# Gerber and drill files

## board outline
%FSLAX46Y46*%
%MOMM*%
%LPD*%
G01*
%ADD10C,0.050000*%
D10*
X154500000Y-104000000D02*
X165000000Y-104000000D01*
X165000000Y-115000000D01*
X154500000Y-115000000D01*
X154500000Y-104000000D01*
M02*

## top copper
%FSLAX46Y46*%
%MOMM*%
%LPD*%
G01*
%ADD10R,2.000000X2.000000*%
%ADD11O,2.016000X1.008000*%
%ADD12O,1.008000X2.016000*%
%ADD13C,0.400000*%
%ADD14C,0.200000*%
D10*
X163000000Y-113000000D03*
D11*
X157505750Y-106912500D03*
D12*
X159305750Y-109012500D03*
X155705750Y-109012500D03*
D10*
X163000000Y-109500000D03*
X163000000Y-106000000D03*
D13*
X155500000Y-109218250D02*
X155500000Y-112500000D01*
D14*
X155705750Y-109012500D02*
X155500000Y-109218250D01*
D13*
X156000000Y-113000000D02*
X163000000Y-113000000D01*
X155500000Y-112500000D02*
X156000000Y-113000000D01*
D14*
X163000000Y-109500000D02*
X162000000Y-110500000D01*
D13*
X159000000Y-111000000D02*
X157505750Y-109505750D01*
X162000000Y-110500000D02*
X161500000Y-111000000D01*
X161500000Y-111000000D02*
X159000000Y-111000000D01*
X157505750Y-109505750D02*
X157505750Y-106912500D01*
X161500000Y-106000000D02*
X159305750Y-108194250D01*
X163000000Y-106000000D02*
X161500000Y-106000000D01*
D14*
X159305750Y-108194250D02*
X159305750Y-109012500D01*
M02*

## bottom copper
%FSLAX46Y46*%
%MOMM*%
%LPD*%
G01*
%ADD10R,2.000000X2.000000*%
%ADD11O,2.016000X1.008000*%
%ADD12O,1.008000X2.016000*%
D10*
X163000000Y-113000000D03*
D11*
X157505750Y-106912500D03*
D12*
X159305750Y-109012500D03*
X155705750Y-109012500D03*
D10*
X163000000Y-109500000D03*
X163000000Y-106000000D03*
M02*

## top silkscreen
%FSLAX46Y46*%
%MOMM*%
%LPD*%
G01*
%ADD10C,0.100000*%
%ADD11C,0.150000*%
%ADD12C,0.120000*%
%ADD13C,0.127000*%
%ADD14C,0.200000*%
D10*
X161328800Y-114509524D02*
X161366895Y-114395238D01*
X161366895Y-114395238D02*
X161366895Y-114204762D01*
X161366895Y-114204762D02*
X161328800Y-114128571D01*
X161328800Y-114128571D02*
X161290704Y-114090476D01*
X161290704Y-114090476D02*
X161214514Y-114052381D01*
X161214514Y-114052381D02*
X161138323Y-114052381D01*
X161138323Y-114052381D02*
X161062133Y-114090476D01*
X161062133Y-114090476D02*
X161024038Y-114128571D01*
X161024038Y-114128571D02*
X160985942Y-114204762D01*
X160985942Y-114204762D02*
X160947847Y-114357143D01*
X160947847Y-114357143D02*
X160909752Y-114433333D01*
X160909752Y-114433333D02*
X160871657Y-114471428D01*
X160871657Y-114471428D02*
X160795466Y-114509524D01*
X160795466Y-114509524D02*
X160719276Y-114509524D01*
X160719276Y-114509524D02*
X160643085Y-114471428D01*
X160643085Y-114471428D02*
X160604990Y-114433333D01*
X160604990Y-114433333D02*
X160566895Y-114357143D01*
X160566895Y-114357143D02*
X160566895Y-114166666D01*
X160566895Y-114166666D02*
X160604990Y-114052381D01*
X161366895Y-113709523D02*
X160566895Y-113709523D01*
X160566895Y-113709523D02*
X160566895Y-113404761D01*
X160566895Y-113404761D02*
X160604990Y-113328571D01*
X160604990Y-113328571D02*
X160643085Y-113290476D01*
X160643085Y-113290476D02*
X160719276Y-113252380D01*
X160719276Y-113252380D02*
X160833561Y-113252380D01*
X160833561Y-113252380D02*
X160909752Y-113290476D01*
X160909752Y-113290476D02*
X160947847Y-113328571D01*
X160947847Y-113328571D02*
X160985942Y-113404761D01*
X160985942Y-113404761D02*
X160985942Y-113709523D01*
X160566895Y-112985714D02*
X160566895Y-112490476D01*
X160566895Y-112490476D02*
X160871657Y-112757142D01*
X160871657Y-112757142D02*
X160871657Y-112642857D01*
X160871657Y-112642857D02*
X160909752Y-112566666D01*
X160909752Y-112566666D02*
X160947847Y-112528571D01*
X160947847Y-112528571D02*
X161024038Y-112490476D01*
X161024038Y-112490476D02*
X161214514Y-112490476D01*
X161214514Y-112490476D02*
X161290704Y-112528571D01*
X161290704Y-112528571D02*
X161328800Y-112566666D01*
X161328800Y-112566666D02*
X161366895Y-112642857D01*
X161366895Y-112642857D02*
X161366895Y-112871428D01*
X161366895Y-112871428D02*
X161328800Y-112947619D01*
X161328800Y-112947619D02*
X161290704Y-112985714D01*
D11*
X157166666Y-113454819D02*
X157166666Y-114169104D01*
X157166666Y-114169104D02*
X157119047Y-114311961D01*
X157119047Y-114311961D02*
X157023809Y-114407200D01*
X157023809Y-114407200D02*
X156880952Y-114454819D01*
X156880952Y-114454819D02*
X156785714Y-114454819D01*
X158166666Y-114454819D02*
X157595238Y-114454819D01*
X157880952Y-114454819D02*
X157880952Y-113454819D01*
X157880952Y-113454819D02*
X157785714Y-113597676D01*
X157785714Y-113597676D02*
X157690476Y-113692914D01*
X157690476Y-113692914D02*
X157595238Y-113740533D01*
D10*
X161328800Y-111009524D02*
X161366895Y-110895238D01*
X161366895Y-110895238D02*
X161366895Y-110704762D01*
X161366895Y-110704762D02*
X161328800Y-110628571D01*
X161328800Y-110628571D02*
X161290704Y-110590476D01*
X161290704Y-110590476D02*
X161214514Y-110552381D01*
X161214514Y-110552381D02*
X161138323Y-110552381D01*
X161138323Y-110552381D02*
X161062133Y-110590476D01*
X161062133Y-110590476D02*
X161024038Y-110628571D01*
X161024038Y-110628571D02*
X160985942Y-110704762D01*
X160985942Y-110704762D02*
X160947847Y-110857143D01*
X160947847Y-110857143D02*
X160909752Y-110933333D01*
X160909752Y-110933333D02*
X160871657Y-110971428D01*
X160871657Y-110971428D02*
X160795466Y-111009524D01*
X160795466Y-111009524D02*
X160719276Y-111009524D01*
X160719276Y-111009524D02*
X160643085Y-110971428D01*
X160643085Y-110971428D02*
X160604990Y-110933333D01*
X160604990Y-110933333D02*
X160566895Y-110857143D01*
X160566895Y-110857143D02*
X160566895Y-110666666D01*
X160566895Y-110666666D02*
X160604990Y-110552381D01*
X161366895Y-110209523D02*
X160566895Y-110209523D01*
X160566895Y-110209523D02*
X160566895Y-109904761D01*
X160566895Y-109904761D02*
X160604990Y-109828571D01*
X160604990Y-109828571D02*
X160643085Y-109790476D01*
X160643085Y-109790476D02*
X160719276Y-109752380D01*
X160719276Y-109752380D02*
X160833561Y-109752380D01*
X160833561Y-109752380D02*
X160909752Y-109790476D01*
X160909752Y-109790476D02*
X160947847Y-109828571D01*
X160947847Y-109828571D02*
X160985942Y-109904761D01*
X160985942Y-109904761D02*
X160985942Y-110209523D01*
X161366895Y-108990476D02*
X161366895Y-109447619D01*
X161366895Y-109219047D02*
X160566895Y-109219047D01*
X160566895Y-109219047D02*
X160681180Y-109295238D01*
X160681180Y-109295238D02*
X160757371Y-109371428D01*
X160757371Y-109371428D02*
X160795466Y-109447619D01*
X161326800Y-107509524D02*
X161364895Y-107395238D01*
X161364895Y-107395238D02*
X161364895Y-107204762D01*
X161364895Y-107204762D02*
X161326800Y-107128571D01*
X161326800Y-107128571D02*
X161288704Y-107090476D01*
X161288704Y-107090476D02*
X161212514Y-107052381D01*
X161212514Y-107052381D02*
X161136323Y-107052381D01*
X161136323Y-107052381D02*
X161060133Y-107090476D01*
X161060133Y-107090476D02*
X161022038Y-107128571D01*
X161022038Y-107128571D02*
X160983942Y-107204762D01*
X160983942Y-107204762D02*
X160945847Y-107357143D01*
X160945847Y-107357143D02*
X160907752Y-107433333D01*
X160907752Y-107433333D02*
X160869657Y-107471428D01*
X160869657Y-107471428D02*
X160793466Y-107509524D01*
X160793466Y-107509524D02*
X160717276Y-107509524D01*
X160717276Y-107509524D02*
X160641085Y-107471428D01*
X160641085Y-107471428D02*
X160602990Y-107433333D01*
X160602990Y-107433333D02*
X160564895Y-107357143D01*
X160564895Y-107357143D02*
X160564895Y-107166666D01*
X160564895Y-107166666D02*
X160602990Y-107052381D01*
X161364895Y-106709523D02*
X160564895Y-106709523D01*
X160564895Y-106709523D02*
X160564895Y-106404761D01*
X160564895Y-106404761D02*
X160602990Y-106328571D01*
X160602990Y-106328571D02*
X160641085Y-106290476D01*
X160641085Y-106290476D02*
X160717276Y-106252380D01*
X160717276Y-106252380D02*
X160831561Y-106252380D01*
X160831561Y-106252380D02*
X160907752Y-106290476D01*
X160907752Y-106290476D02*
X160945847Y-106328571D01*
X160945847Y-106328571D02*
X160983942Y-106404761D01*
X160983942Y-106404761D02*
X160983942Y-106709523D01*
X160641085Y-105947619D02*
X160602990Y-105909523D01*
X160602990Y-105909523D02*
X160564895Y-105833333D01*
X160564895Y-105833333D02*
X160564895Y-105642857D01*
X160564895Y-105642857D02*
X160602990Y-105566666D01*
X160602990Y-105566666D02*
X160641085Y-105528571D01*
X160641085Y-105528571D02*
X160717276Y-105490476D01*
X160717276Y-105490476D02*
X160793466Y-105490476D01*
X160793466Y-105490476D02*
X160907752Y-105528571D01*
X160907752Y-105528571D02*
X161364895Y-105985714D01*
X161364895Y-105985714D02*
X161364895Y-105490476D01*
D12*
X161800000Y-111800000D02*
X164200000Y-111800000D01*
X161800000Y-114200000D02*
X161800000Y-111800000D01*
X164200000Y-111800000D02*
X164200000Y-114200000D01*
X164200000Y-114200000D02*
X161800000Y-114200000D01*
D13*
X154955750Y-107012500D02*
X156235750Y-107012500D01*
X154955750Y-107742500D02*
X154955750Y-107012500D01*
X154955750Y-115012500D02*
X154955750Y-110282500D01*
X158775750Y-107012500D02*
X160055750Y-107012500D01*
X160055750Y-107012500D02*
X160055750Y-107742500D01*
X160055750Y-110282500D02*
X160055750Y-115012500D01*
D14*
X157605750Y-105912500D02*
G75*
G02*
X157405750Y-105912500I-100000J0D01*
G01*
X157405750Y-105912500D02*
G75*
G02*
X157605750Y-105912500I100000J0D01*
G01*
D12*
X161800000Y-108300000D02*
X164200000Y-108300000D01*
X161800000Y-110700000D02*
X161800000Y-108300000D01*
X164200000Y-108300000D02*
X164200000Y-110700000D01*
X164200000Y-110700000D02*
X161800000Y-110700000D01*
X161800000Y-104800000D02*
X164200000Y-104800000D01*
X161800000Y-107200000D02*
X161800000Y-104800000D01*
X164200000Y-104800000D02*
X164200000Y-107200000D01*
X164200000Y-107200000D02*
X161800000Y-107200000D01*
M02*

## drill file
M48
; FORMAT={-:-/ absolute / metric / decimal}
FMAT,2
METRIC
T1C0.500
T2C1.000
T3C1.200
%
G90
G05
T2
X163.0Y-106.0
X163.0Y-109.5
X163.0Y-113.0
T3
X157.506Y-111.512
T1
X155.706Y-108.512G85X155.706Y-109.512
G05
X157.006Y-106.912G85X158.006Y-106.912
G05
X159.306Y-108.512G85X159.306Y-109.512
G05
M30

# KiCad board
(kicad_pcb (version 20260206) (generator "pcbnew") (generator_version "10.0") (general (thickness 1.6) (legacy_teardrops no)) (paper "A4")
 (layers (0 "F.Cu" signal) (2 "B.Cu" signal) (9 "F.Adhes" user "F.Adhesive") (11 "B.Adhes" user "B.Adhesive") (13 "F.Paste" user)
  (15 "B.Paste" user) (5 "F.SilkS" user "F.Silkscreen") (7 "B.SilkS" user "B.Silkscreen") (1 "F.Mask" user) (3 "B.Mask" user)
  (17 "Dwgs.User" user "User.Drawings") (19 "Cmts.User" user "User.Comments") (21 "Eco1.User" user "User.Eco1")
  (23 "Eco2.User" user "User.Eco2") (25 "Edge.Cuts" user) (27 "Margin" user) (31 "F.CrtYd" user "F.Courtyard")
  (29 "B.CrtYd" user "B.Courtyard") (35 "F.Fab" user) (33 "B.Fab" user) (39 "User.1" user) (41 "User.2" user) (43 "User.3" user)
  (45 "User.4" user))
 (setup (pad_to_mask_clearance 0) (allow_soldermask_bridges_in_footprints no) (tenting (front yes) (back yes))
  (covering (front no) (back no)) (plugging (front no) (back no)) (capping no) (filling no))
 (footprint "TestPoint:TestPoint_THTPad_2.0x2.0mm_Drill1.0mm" (layer "F.Cu") (at 163 113)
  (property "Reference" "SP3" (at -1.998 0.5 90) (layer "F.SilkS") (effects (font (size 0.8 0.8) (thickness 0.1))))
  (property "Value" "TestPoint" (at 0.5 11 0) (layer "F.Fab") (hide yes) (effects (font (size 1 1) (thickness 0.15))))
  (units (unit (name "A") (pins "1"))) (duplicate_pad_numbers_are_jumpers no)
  (fp_line (start -1.2 -1.2) (end 1.2 -1.2) (stroke (width 0.12) (type solid)) (layer "F.SilkS"))
  (fp_line (start -1.2 1.2) (end -1.2 -1.2) (stroke (width 0.12) (type solid)) (layer "F.SilkS"))
  (fp_line (start 1.2 -1.2) (end 1.2 1.2) (stroke (width 0.12) (type solid)) (layer "F.SilkS"))
  (fp_line (start 1.2 1.2) (end -1.2 1.2) (stroke (width 0.12) (type solid)) (layer "F.SilkS"))
  (pad "1" thru_hole rect (at 0 0) (size 2 2) (drill 1) (layers "*.Cu" "*.Mask") (remove_unused_layers no) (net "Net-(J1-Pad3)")))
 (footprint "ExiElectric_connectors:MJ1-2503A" (layer "F.Cu") (at 157.50575 111.5125)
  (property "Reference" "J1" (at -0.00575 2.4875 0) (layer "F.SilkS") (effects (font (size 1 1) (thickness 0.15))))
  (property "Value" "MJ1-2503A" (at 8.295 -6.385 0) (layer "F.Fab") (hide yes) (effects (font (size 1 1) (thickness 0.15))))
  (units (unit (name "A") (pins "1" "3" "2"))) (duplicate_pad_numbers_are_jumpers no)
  (fp_line (start -2.55 -4.5) (end -1.27 -4.5) (stroke (width 0.127) (type solid)) (layer "F.SilkS"))
  (fp_line (start -2.55 -3.77) (end -2.55 -4.5) (stroke (width 0.127) (type solid)) (layer "F.SilkS"))
  (fp_line (start -2.55 3.5) (end -2.55 -1.23) (stroke (width 0.127) (type solid)) (layer "F.SilkS"))
  (fp_line (start 1.27 -4.5) (end 2.55 -4.5) (stroke (width 0.127) (type solid)) (layer "F.SilkS"))
  (fp_line (start 2.55 -4.5) (end 2.55 -3.77) (stroke (width 0.127) (type solid)) (layer "F.SilkS"))
  (fp_line (start 2.55 -1.23) (end 2.55 3.5) (stroke (width 0.127) (type solid)) (layer "F.SilkS"))
  (fp_circle (center 0 -5.6) (end 0.1 -5.6) (stroke (width 0.2) (type solid)) (fill no) (layer "F.SilkS"))
  (pad "" np_thru_hole circle (at 0 0) (size 1.2 1.2) (drill 1.2) (layers "*.Cu" "*.Mask"))
  (pad "1" thru_hole oval (at 0 -4.6) (size 2.016 1.008) (drill oval 1.5 0.5) (layers "*.Cu" "*.Mask") (remove_unused_layers no)
   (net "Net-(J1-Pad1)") (solder_mask_margin 0.102))
  (pad "2" thru_hole oval (at 1.8 -2.5) (size 1.008 2.016) (drill oval 0.5 1.5) (layers "*.Cu" "*.Mask") (remove_unused_layers no)
   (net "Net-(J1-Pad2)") (solder_mask_margin 0.102))
  (pad "3" thru_hole oval (at -1.8 -2.5) (size 1.008 2.016) (drill oval 0.5 1.5) (layers "*.Cu" "*.Mask") (remove_unused_layers no)
   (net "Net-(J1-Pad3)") (solder_mask_margin 0.102)))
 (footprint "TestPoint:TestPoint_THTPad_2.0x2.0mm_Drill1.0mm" (layer "F.Cu") (at 163 109.5)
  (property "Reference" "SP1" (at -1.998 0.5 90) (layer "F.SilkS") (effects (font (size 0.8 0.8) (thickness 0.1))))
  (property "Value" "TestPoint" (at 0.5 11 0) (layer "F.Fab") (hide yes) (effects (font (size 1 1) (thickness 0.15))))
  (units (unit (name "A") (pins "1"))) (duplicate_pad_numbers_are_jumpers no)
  (fp_line (start -1.2 -1.2) (end 1.2 -1.2) (stroke (width 0.12) (type solid)) (layer "F.SilkS"))
  (fp_line (start -1.2 1.2) (end -1.2 -1.2) (stroke (width 0.12) (type solid)) (layer "F.SilkS"))
  (fp_line (start 1.2 -1.2) (end 1.2 1.2) (stroke (width 0.12) (type solid)) (layer "F.SilkS"))
  (fp_line (start 1.2 1.2) (end -1.2 1.2) (stroke (width 0.12) (type solid)) (layer "F.SilkS"))
  (pad "1" thru_hole rect (at 0 0) (size 2 2) (drill 1) (layers "*.Cu" "*.Mask") (remove_unused_layers no) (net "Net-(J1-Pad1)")))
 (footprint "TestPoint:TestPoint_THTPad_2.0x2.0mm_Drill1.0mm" (layer "F.Cu") (at 163 106)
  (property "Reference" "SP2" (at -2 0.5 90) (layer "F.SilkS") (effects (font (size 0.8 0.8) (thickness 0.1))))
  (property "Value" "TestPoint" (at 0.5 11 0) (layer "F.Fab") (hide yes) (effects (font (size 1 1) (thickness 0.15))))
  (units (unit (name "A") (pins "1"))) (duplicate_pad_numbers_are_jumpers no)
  (fp_line (start -1.2 -1.2) (end 1.2 -1.2) (stroke (width 0.12) (type solid)) (layer "F.SilkS"))
  (fp_line (start -1.2 1.2) (end -1.2 -1.2) (stroke (width 0.12) (type solid)) (layer "F.SilkS"))
  (fp_line (start 1.2 -1.2) (end 1.2 1.2) (stroke (width 0.12) (type solid)) (layer "F.SilkS"))
  (fp_line (start 1.2 1.2) (end -1.2 1.2) (stroke (width 0.12) (type solid)) (layer "F.SilkS"))
  (pad "1" thru_hole rect (at 0 0) (size 2 2) (drill 1) (layers "*.Cu" "*.Mask") (remove_unused_layers no) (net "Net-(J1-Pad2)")))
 (gr_rect (start 154.5 104) (end 165 115) (stroke (width 0.05) (type default)) (fill no) (layer "Edge.Cuts"))
 (segment (start 155.5 109.21825) (end 155.5 112.5) (width 0.4) (layer "F.Cu") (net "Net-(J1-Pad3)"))
 (segment (start 155.70575 109.0125) (end 155.5 109.21825) (width 0.2) (layer "F.Cu") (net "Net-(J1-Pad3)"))
 (segment (start 156 113) (end 163 113) (width 0.4) (layer "F.Cu") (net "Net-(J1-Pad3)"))
 (segment (start 155.5 112.5) (end 156 113) (width 0.4) (layer "F.Cu") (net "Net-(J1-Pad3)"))
 (segment (start 163 109.5) (end 162 110.5) (width 0.2) (layer "F.Cu") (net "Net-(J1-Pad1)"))
 (segment (start 159 111) (end 157.50575 109.50575) (width 0.4) (layer "F.Cu") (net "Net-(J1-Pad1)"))
 (segment (start 162 110.5) (end 161.5 111) (width 0.4) (layer "F.Cu") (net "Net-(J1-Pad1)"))
 (segment (start 161.5 111) (end 159 111) (width 0.4) (layer "F.Cu") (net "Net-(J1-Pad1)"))
 (segment (start 157.50575 109.50575) (end 157.50575 106.9125) (width 0.4) (layer "F.Cu") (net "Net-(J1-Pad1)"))
 (segment (start 161.5 106) (end 159.30575 108.19425) (width 0.4) (layer "F.Cu") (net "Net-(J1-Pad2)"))
 (segment (start 163 106) (end 161.5 106) (width 0.4) (layer "F.Cu") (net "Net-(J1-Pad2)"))
 (segment (start 159.30575 108.19425) (end 159.30575 109.0125) (width 0.2) (layer "F.Cu") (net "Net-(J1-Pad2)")))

